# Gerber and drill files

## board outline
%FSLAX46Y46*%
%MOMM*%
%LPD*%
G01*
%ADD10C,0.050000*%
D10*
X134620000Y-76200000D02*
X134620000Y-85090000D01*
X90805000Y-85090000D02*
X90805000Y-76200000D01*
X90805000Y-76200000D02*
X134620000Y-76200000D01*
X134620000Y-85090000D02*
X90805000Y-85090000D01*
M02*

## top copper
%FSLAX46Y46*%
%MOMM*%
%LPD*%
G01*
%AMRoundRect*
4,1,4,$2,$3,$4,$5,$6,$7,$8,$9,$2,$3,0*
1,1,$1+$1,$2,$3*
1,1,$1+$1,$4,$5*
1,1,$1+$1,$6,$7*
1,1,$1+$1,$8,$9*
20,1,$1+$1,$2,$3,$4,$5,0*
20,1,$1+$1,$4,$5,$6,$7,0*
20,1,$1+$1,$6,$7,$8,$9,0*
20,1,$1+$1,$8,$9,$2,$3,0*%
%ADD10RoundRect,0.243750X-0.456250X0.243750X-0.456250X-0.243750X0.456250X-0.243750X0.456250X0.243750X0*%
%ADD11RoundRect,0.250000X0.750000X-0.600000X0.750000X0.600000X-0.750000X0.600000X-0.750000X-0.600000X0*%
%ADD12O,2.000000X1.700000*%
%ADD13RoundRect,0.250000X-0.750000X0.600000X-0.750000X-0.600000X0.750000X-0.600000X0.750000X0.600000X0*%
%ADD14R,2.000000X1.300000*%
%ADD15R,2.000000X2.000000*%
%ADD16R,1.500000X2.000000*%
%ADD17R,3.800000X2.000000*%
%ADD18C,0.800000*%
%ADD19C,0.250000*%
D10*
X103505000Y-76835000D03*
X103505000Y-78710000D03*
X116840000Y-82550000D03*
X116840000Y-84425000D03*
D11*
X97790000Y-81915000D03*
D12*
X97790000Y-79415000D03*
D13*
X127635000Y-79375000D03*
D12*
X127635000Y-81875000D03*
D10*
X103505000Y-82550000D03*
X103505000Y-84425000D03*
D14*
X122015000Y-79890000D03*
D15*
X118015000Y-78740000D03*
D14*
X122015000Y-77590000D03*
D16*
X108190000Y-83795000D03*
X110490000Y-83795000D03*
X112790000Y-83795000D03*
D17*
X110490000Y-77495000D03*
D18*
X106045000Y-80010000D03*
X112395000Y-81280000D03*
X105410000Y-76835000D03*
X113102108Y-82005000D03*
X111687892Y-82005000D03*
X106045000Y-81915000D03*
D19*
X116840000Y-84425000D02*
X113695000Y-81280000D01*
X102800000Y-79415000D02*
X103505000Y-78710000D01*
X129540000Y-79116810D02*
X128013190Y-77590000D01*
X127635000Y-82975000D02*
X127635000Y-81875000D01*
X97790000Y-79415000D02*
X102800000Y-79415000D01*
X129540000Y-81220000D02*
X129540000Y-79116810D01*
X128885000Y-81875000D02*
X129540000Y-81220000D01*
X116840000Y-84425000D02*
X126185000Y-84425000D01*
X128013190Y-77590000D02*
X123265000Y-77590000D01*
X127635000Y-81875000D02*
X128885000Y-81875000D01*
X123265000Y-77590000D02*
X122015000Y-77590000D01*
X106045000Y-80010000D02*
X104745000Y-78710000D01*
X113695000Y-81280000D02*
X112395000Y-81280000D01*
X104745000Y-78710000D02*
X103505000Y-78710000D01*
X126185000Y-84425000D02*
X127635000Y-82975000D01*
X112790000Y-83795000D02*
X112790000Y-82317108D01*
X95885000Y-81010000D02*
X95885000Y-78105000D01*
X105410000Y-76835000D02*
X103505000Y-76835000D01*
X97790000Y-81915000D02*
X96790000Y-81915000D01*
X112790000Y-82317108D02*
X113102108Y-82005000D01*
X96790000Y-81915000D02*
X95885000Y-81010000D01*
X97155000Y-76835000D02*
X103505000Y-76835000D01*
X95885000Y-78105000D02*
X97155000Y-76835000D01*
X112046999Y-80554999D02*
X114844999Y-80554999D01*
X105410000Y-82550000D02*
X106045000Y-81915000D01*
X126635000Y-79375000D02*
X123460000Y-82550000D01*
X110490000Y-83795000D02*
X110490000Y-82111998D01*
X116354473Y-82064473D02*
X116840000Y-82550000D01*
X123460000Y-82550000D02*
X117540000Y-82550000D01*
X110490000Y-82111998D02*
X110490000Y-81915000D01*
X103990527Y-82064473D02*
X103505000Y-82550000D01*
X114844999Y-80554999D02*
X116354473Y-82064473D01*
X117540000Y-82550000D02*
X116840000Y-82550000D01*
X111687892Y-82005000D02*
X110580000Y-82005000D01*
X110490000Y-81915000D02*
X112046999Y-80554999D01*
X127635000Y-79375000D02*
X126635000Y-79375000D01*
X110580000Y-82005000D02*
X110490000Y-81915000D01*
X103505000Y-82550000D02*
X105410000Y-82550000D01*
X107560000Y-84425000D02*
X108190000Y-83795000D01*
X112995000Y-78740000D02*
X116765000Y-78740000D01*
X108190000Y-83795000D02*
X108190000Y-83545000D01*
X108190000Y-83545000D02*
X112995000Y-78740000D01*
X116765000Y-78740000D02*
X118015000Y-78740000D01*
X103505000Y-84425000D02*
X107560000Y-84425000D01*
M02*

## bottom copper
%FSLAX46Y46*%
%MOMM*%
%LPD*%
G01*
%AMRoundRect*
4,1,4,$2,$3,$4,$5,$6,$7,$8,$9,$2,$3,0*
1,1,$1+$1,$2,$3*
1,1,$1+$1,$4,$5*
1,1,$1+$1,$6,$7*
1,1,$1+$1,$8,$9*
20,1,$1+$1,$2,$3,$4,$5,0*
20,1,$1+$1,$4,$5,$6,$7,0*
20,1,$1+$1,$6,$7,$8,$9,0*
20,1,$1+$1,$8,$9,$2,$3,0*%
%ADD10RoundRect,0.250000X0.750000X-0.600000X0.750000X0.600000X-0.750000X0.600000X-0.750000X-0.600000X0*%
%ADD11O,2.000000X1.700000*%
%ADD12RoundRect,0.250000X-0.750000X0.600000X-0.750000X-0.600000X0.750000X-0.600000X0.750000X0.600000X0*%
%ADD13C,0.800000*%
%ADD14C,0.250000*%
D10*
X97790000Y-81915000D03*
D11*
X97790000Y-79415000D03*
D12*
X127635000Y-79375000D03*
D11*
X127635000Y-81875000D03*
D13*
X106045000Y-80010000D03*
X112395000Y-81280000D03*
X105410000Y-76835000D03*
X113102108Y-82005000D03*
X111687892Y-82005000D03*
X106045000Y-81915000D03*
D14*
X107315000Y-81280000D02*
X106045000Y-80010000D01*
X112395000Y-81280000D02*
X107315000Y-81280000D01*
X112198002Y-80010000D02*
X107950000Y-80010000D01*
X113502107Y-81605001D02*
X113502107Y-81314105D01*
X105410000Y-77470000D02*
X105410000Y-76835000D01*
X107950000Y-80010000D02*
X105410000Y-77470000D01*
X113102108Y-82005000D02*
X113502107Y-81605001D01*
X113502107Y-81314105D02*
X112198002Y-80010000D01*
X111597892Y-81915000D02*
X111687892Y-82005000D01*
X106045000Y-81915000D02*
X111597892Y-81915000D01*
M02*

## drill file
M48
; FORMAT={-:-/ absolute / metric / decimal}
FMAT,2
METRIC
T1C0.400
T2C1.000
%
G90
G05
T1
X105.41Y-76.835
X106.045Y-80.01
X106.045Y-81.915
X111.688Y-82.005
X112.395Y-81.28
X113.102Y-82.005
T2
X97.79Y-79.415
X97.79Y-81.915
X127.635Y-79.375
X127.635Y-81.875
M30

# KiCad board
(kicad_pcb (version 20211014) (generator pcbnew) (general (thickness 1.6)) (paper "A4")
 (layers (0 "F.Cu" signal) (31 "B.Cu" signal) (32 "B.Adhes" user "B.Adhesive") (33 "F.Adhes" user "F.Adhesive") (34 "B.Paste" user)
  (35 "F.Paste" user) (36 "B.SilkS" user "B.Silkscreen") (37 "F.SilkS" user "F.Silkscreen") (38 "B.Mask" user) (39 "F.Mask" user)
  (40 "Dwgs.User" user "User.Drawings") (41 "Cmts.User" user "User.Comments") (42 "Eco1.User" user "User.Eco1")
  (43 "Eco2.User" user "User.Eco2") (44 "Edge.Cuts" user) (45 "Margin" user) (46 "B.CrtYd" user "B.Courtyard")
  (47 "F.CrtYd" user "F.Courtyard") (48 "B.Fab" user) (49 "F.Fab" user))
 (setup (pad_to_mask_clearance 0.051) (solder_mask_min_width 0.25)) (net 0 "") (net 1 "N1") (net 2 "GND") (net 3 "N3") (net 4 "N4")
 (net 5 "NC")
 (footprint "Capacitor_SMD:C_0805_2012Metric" (layer "F.Cu") (at 103.505 77.7725 -90)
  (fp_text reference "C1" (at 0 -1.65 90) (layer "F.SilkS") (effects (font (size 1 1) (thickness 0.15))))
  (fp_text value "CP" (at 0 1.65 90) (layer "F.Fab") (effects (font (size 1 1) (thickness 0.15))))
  (pad "1" smd roundrect locked (at -0.9375 0 270) (size 0.975 1.4) (layers "F.Cu" "F.Paste" "F.Mask") (roundrect_rratio 0.25) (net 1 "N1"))
  (pad "2" smd roundrect locked (at 0.9375 0 270) (size 0.975 1.4) (layers "F.Cu" "F.Paste" "F.Mask") (roundrect_rratio 0.25) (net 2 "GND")))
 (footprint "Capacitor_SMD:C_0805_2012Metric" (layer "F.Cu") (at 116.84 83.4875 -90)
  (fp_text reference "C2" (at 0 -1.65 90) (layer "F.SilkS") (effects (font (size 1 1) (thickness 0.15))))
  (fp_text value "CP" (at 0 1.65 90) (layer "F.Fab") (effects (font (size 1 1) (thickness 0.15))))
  (pad "1" smd roundrect locked (at -0.9375 0 270) (size 0.975 1.4) (layers "F.Cu" "F.Paste" "F.Mask") (roundrect_rratio 0.25) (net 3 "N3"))
  (pad "2" smd roundrect locked (at 0.9375 0 270) (size 0.975 1.4) (layers "F.Cu" "F.Paste" "F.Mask") (roundrect_rratio 0.25) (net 2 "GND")))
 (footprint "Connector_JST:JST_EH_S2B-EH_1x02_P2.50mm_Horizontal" (layer "F.Cu") (at 97.79 81.915 90)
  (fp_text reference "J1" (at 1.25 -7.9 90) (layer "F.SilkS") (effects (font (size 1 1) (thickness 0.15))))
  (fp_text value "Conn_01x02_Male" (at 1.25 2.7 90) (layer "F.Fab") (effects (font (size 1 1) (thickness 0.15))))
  (pad "1" thru_hole roundrect locked (at 0 0 90) (size 1.7 2) (drill 1) (layers *.Cu *.Mask) (roundrect_rratio 0.147059) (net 1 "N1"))
  (pad "2" thru_hole oval locked (at 2.5 0 90) (size 1.7 2) (drill 1) (layers *.Cu *.Mask) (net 2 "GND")))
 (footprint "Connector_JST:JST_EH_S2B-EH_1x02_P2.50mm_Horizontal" (layer "F.Cu") (at 127.635 79.375 -90)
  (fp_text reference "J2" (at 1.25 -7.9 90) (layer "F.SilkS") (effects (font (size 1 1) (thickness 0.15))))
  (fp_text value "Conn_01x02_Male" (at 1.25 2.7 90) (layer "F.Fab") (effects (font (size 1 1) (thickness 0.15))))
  (pad "1" thru_hole roundrect locked (at 0 0 270) (size 1.7 2) (drill 1) (layers *.Cu *.Mask) (roundrect_rratio 0.147059) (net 3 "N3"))
  (pad "2" thru_hole oval locked (at 2.5 0 270) (size 1.7 2) (drill 1) (layers *.Cu *.Mask) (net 2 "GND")))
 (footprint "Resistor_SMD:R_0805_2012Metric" (layer "F.Cu") (at 103.505 83.4875 -90)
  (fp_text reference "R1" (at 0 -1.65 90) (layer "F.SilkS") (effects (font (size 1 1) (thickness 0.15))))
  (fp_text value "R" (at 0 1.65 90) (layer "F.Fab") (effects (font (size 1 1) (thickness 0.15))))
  (pad "1" smd roundrect locked (at -0.9375 0 270) (size 0.975 1.4) (layers "F.Cu" "F.Paste" "F.Mask") (roundrect_rratio 0.25) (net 3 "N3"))
  (pad "2" smd roundrect locked (at 0.9375 0 270) (size 0.975 1.4) (layers "F.Cu" "F.Paste" "F.Mask") (roundrect_rratio 0.25) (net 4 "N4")))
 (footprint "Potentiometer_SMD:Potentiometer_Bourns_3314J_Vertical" (layer "F.Cu") (at 120.015 78.74 -90)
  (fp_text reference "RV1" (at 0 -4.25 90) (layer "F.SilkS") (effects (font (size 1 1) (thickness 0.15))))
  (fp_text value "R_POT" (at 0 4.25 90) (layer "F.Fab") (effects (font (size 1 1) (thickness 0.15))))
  (pad "1" smd rect locked (at 1.15 -2 270) (size 1.3 2) (layers "F.Cu" "F.Paste" "F.Mask") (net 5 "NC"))
  (pad "2" smd rect locked (at 0 2 270) (size 2 2) (layers "F.Cu" "F.Paste" "F.Mask") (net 4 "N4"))
  (pad "3" smd rect locked (at -1.15 -2 270) (size 1.3 2) (layers "F.Cu" "F.Paste" "F.Mask") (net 2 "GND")))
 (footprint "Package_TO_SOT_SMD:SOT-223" (layer "F.Cu") (at 110.49 80.645 90)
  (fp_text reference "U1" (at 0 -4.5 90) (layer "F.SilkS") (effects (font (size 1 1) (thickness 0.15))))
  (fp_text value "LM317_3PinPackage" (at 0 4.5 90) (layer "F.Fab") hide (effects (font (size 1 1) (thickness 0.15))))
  (pad "1" smd rect locked (at -3.15 -2.3 90) (size 2 1.5) (layers "F.Cu" "F.Paste" "F.Mask") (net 4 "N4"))
  (pad "2" smd rect locked (at -3.15 0 90) (size 2 1.5) (layers "F.Cu" "F.Paste" "F.Mask") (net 3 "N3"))
  (pad "3" smd rect locked (at -3.15 2.3 90) (size 2 1.5) (layers "F.Cu" "F.Paste" "F.Mask") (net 1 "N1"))
  (pad "4" smd rect locked (at 3.15 0 90) (size 2 3.8) (layers "F.Cu" "F.Paste" "F.Mask")))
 (gr_line (start 134.62 76.2) (end 134.62 85.09) (layer "Edge.Cuts") (width 0.05))
 (gr_line (start 90.805 85.09) (end 90.805 76.2) (layer "Edge.Cuts") (width 0.05))
 (gr_line (start 90.805 76.2) (end 134.62 76.2) (layer "Edge.Cuts") (width 0.05))
 (gr_line (start 134.62 85.09) (end 90.805 85.09) (layer "Edge.Cuts") (width 0.05))
 (segment (start 116.84 84.425) (end 113.695 81.28) (width 0.25) (layer "F.Cu") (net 2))
 (segment (start 102.8 79.415) (end 103.505 78.71) (width 0.25) (layer "F.Cu") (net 2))
 (segment (start 129.54 79.11681) (end 128.01319 77.59) (width 0.25) (layer "F.Cu") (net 2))
 (segment (start 127.635 82.975) (end 127.635 81.875) (width 0.25) (layer "F.Cu") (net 2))
 (segment (start 97.79 79.415) (end 102.8 79.415) (width 0.25) (layer "F.Cu") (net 2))
 (segment (start 129.54 81.22) (end 129.54 79.11681) (width 0.25) (layer "F.Cu") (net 2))
 (segment (start 128.885 81.875) (end 129.54 81.22) (width 0.25) (layer "F.Cu") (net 2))
 (segment (start 116.84 84.425) (end 126.185 84.425) (width 0.25) (layer "F.Cu") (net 2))
 (segment (start 128.01319 77.59) (end 123.265 77.59) (width 0.25) (layer "F.Cu") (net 2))
 (segment (start 127.635 81.875) (end 128.885 81.875) (width 0.25) (layer "F.Cu") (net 2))
 (segment (start 123.265 77.59) (end 122.015 77.59) (width 0.25) (layer "F.Cu") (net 2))
 (segment (start 106.045 80.01) (end 104.745 78.71) (width 0.25) (layer "F.Cu") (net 2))
 (segment (start 113.695 81.28) (end 112.395 81.28) (width 0.25) (layer "F.Cu") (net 2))
 (segment (start 104.745 78.71) (end 103.505 78.71) (width 0.25) (layer "F.Cu") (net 2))
 (segment (start 126.185 84.425) (end 127.635 82.975) (width 0.25) (layer "F.Cu") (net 2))
 (via (at 106.045 80.01) (size 0.8) (drill 0.4) (layers "F.Cu" "B.Cu") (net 2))
 (via (at 112.395 81.28) (size 0.8) (drill 0.4) (layers "F.Cu" "B.Cu") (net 2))
 (segment (start 107.315 81.28) (end 106.045 80.01) (width 0.25) (layer "B.Cu") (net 2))
 (segment (start 112.395 81.28) (end 107.315 81.28) (width 0.25) (layer "B.Cu") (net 2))
 (segment (start 112.79 83.795) (end 112.79 82.317108) (width 0.25) (layer "F.Cu") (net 1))
 (segment (start 95.885 81.01) (end 95.885 78.105) (width 0.25) (layer "F.Cu") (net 1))
 (segment (start 105.41 76.835) (end 103.505 76.835) (width 0.25) (layer "F.Cu") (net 1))
 (segment (start 97.79 81.915) (end 96.79 81.915) (width 0.25) (layer "F.Cu") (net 1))
 (segment (start 112.79 82.317108) (end 113.102108 82.005) (width 0.25) (layer "F.Cu") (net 1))
 (segment (start 96.79 81.915) (end 95.885 81.01) (width 0.25) (layer "F.Cu") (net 1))
 (segment (start 97.155 76.835) (end 103.505 76.835) (width 0.25) (layer "F.Cu") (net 1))
 (segment (start 95.885 78.105) (end 97.155 76.835) (width 0.25) (layer "F.Cu") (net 1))
 (via (at 105.41 76.835) (size 0.8) (drill 0.4) (layers "F.Cu" "B.Cu") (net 1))
 (via (at 113.102108 82.005) (size 0.8) (drill 0.4) (layers "F.Cu" "B.Cu") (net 1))
 (segment (start 112.198002 80.01) (end 107.95 80.01) (width 0.25) (layer "B.Cu") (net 1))
 (segment (start 113.502107 81.605001) (end 113.502107 81.314105) (width 0.25) (layer "B.Cu") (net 1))
 (segment (start 105.41 77.47) (end 105.41 76.835) (width 0.25) (layer "B.Cu") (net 1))
 (segment (start 107.95 80.01) (end 105.41 77.47) (width 0.25) (layer "B.Cu") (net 1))
 (segment (start 113.102108 82.005) (end 113.502107 81.605001) (width 0.25) (layer "B.Cu") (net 1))
 (segment (start 113.502107 81.314105) (end 112.198002 80.01) (width 0.25) (layer "B.Cu") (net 1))
 (segment (start 112.046999 80.554999) (end 114.844999 80.554999) (width 0.25) (layer "F.Cu") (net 3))
 (segment (start 105.41 82.55) (end 106.045 81.915) (width 0.25) (layer "F.Cu") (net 3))
 (segment (start 126.635 79.375) (end 123.46 82.55) (width 0.25) (layer "F.Cu") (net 3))
 (segment (start 110.49 83.795) (end 110.49 82.111998) (width 0.25) (layer "F.Cu") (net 3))
 (segment (start 116.354473 82.064473) (end 116.84 82.55) (width 0.25) (layer "F.Cu") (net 3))
 (segment (start 123.46 82.55) (end 117.54 82.55) (width 0.25) (layer "F.Cu") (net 3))
 (segment (start 110.49 82.111998) (end 110.49 81.915) (width 0.25) (layer "F.Cu") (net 3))
 (segment (start 103.990527 82.064473) (end 103.505 82.55) (width 0.25) (layer "F.Cu") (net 3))
 (segment (start 114.844999 80.554999) (end 116.354473 82.064473) (width 0.25) (layer "F.Cu") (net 3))
 (segment (start 117.54 82.55) (end 116.84 82.55) (width 0.25) (layer "F.Cu") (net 3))
 (segment (start 111.687892 82.005) (end 110.58 82.005) (width 0.25) (layer "F.Cu") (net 3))
 (segment (start 110.49 81.915) (end 112.046999 80.554999) (width 0.25) (layer "F.Cu") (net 3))
 (segment (start 127.635 79.375) (end 126.635 79.375) (width 0.25) (layer "F.Cu") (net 3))
 (segment (start 110.58 82.005) (end 110.49 81.915) (width 0.25) (layer "F.Cu") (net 3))
 (segment (start 103.505 82.55) (end 105.41 82.55) (width 0.25) (layer "F.Cu") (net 3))
 (via (at 111.687892 82.005) (size 0.8) (drill 0.4) (layers "F.Cu" "B.Cu") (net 3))
 (via (at 106.045 81.915) (size 0.8) (drill 0.4) (layers "F.Cu" "B.Cu") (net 3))
 (segment (start 111.597892 81.915) (end 111.687892 82.005) (width 0.25) (layer "B.Cu") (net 3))
 (segment (start 106.045 81.915) (end 111.597892 81.915) (width 0.25) (layer "B.Cu") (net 3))
 (segment (start 107.56 84.425) (end 108.19 83.795) (width 0.25) (layer "F.Cu") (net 4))
 (segment (start 112.995 78.74) (end 116.765 78.74) (width 0.25) (layer "F.Cu") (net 4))
 (segment (start 108.19 83.795) (end 108.19 83.545) (width 0.25) (layer "F.Cu") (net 4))
 (segment (start 108.19 83.545) (end 112.995 78.74) (width 0.25) (layer "F.Cu") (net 4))
 (segment (start 116.765 78.74) (end 118.015 78.74) (width 0.25) (layer "F.Cu") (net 4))
 (segment (start 103.505 84.425) (end 107.56 84.425) (width 0.25) (layer "F.Cu") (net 4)))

